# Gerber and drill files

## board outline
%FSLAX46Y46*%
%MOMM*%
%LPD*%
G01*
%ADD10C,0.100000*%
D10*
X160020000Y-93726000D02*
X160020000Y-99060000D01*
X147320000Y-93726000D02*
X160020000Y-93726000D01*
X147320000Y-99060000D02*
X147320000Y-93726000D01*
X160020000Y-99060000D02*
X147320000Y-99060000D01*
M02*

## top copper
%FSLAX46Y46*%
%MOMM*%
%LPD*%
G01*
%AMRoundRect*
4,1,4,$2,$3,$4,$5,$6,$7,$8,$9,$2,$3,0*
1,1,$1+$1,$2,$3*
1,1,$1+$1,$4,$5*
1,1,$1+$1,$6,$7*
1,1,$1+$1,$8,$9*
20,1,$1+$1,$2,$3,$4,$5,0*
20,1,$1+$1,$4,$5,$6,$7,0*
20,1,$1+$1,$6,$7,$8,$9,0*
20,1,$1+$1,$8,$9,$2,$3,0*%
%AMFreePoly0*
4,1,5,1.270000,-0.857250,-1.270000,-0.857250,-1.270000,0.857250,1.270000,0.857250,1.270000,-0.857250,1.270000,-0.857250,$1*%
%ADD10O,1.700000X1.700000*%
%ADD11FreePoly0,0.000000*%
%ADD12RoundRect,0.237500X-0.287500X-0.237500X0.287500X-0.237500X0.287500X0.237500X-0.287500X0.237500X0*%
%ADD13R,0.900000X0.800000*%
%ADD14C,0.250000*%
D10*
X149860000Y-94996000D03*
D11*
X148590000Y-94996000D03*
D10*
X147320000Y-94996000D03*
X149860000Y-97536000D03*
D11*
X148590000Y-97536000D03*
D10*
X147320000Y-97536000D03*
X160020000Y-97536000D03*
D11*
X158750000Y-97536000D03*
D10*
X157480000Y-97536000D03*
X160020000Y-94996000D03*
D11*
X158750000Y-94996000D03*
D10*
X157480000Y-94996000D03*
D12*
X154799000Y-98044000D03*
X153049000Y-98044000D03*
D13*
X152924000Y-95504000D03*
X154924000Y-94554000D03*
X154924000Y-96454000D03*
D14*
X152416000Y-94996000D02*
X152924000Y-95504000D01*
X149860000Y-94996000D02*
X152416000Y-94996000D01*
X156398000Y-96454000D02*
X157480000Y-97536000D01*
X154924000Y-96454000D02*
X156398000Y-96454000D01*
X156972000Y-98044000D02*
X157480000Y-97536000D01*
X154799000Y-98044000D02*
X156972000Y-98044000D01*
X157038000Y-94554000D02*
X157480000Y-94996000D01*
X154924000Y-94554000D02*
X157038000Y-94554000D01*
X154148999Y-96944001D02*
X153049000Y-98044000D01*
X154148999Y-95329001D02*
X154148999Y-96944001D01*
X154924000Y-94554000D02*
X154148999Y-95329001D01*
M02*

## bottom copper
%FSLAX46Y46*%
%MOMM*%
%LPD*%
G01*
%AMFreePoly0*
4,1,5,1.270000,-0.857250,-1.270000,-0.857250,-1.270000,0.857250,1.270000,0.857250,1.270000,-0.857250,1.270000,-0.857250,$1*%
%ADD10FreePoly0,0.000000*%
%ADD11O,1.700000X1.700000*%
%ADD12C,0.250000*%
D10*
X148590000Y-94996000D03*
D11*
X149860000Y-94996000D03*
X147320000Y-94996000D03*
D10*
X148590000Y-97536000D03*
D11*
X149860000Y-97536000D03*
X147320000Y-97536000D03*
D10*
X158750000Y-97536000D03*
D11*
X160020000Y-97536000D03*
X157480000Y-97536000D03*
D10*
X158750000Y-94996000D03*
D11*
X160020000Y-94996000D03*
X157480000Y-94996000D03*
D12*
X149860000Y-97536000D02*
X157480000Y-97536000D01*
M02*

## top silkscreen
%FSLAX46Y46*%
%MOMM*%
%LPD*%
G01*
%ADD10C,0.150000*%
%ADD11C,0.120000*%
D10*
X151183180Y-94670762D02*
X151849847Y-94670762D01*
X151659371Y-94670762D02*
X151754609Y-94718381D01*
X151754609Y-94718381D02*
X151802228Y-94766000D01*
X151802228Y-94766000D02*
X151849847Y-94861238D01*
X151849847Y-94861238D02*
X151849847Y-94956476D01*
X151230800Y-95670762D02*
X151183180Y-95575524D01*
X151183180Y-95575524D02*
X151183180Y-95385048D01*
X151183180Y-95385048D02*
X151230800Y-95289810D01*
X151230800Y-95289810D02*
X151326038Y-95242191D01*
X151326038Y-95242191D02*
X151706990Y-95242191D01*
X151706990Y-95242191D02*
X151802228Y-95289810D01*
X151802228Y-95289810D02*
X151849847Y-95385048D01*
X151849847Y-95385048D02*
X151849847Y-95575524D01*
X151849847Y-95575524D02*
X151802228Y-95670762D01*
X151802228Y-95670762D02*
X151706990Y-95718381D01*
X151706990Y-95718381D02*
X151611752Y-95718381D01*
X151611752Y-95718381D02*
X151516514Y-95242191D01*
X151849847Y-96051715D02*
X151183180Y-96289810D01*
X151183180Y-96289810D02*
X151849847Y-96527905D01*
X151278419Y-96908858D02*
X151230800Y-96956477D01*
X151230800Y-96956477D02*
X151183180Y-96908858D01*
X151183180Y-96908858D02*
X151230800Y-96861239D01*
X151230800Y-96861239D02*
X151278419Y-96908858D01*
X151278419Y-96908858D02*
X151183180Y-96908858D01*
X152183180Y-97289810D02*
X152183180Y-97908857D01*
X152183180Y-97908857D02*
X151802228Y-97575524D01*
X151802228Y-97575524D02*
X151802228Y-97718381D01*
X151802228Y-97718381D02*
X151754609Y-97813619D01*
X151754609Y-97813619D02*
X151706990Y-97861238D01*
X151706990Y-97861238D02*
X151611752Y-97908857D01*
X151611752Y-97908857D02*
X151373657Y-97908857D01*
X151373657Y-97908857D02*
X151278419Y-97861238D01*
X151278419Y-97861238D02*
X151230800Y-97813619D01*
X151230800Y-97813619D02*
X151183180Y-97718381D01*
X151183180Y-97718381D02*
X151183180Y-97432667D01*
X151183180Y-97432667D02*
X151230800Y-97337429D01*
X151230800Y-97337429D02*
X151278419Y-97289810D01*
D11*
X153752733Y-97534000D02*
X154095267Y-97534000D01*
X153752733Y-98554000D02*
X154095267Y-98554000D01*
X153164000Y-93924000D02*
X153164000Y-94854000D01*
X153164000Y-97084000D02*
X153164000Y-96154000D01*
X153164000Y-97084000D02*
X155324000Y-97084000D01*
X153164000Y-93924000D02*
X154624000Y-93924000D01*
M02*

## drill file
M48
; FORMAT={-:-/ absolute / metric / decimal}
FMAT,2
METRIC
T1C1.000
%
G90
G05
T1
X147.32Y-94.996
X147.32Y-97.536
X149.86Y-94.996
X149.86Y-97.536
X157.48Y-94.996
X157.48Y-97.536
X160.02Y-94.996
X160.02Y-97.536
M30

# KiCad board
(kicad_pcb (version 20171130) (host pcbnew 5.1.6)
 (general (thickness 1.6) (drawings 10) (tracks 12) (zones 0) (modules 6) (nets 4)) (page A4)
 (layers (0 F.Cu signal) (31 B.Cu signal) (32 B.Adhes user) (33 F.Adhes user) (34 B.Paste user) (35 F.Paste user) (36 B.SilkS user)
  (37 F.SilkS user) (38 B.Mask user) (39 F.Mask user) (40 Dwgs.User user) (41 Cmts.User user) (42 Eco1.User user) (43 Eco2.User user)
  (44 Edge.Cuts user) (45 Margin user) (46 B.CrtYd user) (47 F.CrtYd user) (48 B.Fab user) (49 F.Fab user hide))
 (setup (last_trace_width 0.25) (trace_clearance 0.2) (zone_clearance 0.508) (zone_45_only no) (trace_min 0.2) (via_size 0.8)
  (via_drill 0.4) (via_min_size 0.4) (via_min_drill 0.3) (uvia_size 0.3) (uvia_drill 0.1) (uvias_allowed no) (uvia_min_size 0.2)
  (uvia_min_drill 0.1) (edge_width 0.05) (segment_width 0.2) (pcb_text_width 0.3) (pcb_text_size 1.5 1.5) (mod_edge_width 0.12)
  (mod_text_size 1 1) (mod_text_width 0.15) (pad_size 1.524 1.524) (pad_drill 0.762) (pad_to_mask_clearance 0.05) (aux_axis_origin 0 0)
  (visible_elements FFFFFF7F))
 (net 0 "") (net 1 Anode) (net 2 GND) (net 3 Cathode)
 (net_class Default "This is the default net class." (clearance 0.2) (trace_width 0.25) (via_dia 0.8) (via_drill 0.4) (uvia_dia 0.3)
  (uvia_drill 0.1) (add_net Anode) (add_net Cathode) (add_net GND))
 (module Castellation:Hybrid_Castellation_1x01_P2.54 (layer F.Cu) (at 148.59 94.996)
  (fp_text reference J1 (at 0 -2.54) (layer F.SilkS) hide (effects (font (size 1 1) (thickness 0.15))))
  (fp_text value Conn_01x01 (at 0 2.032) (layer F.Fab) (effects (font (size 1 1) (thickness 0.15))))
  (pad 1 connect custom (at 0 0) (size 2.54 1.7145) (layers B.Cu B.Mask) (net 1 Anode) (zone_connect 0)
   (options (clearance outline) (anchor rect)) (primitives))
  (pad 1 thru_hole oval (at 1.27 0) (size 1.7 1.7) (drill 1) (layers *.Cu *.Mask) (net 1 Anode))
  (pad 1 connect custom (at 0 0) (size 2.54 1.7145) (layers F.Cu F.Mask) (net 1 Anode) (zone_connect 0)
   (options (clearance outline) (anchor rect)) (primitives))
  (pad 1 thru_hole oval (at -1.27 0) (size 1.7 1.7) (drill 1) (layers *.Cu *.Mask) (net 1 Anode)))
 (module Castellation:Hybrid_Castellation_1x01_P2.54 (layer F.Cu) (at 148.59 97.536)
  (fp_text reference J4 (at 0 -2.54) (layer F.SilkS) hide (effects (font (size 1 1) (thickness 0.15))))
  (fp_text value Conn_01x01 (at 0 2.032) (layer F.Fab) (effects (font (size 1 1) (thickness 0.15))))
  (pad 1 connect custom (at 0 0) (size 2.54 1.7145) (layers B.Cu B.Mask) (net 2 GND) (zone_connect 0)
   (options (clearance outline) (anchor rect)) (primitives))
  (pad 1 thru_hole oval (at 1.27 0) (size 1.7 1.7) (drill 1) (layers *.Cu *.Mask) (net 2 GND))
  (pad 1 connect custom (at 0 0) (size 2.54 1.7145) (layers F.Cu F.Mask) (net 2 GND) (zone_connect 0)
   (options (clearance outline) (anchor rect)) (primitives))
  (pad 1 thru_hole oval (at -1.27 0) (size 1.7 1.7) (drill 1) (layers *.Cu *.Mask) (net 2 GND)))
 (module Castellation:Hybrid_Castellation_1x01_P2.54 (layer F.Cu) (at 158.75 97.536)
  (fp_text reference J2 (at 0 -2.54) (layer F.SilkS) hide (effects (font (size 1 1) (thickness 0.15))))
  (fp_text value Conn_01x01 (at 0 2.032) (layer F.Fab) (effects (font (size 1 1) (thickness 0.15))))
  (pad 1 connect custom (at 0 0) (size 2.54 1.7145) (layers B.Cu B.Mask) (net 2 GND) (zone_connect 0)
   (options (clearance outline) (anchor rect)) (primitives))
  (pad 1 thru_hole oval (at 1.27 0) (size 1.7 1.7) (drill 1) (layers *.Cu *.Mask) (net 2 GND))
  (pad 1 connect custom (at 0 0) (size 2.54 1.7145) (layers F.Cu F.Mask) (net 2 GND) (zone_connect 0)
   (options (clearance outline) (anchor rect)) (primitives))
  (pad 1 thru_hole oval (at -1.27 0) (size 1.7 1.7) (drill 1) (layers *.Cu *.Mask) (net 2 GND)))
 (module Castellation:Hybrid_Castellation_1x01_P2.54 (layer F.Cu) (at 158.75 94.996)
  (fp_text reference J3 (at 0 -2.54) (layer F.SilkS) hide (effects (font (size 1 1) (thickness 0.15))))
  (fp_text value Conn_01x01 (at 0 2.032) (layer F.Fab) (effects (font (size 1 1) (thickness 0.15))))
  (pad 1 connect custom (at 0 0) (size 2.54 1.7145) (layers B.Cu B.Mask) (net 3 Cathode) (zone_connect 0)
   (options (clearance outline) (anchor rect)) (primitives))
  (pad 1 thru_hole oval (at 1.27 0) (size 1.7 1.7) (drill 1) (layers *.Cu *.Mask) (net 3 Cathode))
  (pad 1 connect custom (at 0 0) (size 2.54 1.7145) (layers F.Cu F.Mask) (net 3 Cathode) (zone_connect 0)
   (options (clearance outline) (anchor rect)) (primitives))
  (pad 1 thru_hole oval (at -1.27 0) (size 1.7 1.7) (drill 1) (layers *.Cu *.Mask) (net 3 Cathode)))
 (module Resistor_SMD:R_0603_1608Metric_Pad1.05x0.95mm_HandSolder (layer F.Cu) (at 153.924 98.044)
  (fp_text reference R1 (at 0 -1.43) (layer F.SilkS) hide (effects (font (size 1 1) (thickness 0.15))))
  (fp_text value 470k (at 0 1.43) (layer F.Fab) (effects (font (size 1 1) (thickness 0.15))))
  (fp_line (start -0.171267 -0.51) (end 0.171267 -0.51) (layer F.SilkS) (width 0.12))
  (fp_line (start -0.171267 0.51) (end 0.171267 0.51) (layer F.SilkS) (width 0.12))
  (pad 2 smd roundrect (at 0.875 0) (size 1.05 0.95) (layers F.Cu F.Paste F.Mask) (roundrect_rratio 0.25) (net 2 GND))
  (pad 1 smd roundrect (at -0.875 0) (size 1.05 0.95) (layers F.Cu F.Paste F.Mask) (roundrect_rratio 0.25) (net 3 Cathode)))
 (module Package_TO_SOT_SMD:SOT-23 (layer F.Cu) (at 153.924 95.504 180)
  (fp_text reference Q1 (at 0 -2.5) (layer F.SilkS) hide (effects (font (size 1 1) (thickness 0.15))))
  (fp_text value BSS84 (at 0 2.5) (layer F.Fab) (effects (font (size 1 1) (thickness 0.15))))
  (fp_line (start 0.76 1.58) (end 0.76 0.65) (layer F.SilkS) (width 0.12))
  (fp_line (start 0.76 -1.58) (end 0.76 -0.65) (layer F.SilkS) (width 0.12))
  (fp_line (start 0.76 -1.58) (end -1.4 -1.58) (layer F.SilkS) (width 0.12))
  (fp_line (start 0.76 1.58) (end -0.7 1.58) (layer F.SilkS) (width 0.12))
  (pad 3 smd rect (at 1 0 180) (size 0.9 0.8) (layers F.Cu F.Paste F.Mask) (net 1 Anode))
  (pad 2 smd rect (at -1 0.95 180) (size 0.9 0.8) (layers F.Cu F.Paste F.Mask) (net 3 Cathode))
  (pad 1 smd rect (at -1 -0.95 180) (size 0.9 0.8) (layers F.Cu F.Paste F.Mask) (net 2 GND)))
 (gr_line (start 160.02 93.726) (end 160.02 99.06) (layer Edge.Cuts) (width 0.1))
 (gr_line (start 147.32 93.726) (end 160.02 93.726) (layer Edge.Cuts) (width 0.1))
 (gr_line (start 147.32 99.06) (end 147.32 93.726) (layer Edge.Cuts) (width 0.1))
 (gr_line (start 160.02 99.06) (end 147.32 99.06) (layer Edge.Cuts) (width 0.1))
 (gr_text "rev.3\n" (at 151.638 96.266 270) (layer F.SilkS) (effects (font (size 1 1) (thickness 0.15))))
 (segment (start 152.416 94.996) (end 152.924 95.504) (width 0.25) (layer F.Cu) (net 1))
 (segment (start 149.86 94.996) (end 152.416 94.996) (width 0.25) (layer F.Cu) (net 1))
 (segment (start 156.398 96.454) (end 157.48 97.536) (width 0.25) (layer F.Cu) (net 2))
 (segment (start 154.924 96.454) (end 156.398 96.454) (width 0.25) (layer F.Cu) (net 2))
 (segment (start 156.972 98.044) (end 157.48 97.536) (width 0.25) (layer F.Cu) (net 2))
 (segment (start 154.799 98.044) (end 156.972 98.044) (width 0.25) (layer F.Cu) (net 2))
 (segment (start 149.86 97.536) (end 157.48 97.536) (width 0.25) (layer B.Cu) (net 2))
 (segment (start 157.038 94.554) (end 157.48 94.996) (width 0.25) (layer F.Cu) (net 3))
 (segment (start 154.924 94.554) (end 157.038 94.554) (width 0.25) (layer F.Cu) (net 3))
 (segment (start 154.148999 96.944001) (end 153.049 98.044) (width 0.25) (layer F.Cu) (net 3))
 (segment (start 154.148999 95.329001) (end 154.148999 96.944001) (width 0.25) (layer F.Cu) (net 3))
 (segment (start 154.924 94.554) (end 154.148999 95.329001) (width 0.25) (layer F.Cu) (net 3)))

